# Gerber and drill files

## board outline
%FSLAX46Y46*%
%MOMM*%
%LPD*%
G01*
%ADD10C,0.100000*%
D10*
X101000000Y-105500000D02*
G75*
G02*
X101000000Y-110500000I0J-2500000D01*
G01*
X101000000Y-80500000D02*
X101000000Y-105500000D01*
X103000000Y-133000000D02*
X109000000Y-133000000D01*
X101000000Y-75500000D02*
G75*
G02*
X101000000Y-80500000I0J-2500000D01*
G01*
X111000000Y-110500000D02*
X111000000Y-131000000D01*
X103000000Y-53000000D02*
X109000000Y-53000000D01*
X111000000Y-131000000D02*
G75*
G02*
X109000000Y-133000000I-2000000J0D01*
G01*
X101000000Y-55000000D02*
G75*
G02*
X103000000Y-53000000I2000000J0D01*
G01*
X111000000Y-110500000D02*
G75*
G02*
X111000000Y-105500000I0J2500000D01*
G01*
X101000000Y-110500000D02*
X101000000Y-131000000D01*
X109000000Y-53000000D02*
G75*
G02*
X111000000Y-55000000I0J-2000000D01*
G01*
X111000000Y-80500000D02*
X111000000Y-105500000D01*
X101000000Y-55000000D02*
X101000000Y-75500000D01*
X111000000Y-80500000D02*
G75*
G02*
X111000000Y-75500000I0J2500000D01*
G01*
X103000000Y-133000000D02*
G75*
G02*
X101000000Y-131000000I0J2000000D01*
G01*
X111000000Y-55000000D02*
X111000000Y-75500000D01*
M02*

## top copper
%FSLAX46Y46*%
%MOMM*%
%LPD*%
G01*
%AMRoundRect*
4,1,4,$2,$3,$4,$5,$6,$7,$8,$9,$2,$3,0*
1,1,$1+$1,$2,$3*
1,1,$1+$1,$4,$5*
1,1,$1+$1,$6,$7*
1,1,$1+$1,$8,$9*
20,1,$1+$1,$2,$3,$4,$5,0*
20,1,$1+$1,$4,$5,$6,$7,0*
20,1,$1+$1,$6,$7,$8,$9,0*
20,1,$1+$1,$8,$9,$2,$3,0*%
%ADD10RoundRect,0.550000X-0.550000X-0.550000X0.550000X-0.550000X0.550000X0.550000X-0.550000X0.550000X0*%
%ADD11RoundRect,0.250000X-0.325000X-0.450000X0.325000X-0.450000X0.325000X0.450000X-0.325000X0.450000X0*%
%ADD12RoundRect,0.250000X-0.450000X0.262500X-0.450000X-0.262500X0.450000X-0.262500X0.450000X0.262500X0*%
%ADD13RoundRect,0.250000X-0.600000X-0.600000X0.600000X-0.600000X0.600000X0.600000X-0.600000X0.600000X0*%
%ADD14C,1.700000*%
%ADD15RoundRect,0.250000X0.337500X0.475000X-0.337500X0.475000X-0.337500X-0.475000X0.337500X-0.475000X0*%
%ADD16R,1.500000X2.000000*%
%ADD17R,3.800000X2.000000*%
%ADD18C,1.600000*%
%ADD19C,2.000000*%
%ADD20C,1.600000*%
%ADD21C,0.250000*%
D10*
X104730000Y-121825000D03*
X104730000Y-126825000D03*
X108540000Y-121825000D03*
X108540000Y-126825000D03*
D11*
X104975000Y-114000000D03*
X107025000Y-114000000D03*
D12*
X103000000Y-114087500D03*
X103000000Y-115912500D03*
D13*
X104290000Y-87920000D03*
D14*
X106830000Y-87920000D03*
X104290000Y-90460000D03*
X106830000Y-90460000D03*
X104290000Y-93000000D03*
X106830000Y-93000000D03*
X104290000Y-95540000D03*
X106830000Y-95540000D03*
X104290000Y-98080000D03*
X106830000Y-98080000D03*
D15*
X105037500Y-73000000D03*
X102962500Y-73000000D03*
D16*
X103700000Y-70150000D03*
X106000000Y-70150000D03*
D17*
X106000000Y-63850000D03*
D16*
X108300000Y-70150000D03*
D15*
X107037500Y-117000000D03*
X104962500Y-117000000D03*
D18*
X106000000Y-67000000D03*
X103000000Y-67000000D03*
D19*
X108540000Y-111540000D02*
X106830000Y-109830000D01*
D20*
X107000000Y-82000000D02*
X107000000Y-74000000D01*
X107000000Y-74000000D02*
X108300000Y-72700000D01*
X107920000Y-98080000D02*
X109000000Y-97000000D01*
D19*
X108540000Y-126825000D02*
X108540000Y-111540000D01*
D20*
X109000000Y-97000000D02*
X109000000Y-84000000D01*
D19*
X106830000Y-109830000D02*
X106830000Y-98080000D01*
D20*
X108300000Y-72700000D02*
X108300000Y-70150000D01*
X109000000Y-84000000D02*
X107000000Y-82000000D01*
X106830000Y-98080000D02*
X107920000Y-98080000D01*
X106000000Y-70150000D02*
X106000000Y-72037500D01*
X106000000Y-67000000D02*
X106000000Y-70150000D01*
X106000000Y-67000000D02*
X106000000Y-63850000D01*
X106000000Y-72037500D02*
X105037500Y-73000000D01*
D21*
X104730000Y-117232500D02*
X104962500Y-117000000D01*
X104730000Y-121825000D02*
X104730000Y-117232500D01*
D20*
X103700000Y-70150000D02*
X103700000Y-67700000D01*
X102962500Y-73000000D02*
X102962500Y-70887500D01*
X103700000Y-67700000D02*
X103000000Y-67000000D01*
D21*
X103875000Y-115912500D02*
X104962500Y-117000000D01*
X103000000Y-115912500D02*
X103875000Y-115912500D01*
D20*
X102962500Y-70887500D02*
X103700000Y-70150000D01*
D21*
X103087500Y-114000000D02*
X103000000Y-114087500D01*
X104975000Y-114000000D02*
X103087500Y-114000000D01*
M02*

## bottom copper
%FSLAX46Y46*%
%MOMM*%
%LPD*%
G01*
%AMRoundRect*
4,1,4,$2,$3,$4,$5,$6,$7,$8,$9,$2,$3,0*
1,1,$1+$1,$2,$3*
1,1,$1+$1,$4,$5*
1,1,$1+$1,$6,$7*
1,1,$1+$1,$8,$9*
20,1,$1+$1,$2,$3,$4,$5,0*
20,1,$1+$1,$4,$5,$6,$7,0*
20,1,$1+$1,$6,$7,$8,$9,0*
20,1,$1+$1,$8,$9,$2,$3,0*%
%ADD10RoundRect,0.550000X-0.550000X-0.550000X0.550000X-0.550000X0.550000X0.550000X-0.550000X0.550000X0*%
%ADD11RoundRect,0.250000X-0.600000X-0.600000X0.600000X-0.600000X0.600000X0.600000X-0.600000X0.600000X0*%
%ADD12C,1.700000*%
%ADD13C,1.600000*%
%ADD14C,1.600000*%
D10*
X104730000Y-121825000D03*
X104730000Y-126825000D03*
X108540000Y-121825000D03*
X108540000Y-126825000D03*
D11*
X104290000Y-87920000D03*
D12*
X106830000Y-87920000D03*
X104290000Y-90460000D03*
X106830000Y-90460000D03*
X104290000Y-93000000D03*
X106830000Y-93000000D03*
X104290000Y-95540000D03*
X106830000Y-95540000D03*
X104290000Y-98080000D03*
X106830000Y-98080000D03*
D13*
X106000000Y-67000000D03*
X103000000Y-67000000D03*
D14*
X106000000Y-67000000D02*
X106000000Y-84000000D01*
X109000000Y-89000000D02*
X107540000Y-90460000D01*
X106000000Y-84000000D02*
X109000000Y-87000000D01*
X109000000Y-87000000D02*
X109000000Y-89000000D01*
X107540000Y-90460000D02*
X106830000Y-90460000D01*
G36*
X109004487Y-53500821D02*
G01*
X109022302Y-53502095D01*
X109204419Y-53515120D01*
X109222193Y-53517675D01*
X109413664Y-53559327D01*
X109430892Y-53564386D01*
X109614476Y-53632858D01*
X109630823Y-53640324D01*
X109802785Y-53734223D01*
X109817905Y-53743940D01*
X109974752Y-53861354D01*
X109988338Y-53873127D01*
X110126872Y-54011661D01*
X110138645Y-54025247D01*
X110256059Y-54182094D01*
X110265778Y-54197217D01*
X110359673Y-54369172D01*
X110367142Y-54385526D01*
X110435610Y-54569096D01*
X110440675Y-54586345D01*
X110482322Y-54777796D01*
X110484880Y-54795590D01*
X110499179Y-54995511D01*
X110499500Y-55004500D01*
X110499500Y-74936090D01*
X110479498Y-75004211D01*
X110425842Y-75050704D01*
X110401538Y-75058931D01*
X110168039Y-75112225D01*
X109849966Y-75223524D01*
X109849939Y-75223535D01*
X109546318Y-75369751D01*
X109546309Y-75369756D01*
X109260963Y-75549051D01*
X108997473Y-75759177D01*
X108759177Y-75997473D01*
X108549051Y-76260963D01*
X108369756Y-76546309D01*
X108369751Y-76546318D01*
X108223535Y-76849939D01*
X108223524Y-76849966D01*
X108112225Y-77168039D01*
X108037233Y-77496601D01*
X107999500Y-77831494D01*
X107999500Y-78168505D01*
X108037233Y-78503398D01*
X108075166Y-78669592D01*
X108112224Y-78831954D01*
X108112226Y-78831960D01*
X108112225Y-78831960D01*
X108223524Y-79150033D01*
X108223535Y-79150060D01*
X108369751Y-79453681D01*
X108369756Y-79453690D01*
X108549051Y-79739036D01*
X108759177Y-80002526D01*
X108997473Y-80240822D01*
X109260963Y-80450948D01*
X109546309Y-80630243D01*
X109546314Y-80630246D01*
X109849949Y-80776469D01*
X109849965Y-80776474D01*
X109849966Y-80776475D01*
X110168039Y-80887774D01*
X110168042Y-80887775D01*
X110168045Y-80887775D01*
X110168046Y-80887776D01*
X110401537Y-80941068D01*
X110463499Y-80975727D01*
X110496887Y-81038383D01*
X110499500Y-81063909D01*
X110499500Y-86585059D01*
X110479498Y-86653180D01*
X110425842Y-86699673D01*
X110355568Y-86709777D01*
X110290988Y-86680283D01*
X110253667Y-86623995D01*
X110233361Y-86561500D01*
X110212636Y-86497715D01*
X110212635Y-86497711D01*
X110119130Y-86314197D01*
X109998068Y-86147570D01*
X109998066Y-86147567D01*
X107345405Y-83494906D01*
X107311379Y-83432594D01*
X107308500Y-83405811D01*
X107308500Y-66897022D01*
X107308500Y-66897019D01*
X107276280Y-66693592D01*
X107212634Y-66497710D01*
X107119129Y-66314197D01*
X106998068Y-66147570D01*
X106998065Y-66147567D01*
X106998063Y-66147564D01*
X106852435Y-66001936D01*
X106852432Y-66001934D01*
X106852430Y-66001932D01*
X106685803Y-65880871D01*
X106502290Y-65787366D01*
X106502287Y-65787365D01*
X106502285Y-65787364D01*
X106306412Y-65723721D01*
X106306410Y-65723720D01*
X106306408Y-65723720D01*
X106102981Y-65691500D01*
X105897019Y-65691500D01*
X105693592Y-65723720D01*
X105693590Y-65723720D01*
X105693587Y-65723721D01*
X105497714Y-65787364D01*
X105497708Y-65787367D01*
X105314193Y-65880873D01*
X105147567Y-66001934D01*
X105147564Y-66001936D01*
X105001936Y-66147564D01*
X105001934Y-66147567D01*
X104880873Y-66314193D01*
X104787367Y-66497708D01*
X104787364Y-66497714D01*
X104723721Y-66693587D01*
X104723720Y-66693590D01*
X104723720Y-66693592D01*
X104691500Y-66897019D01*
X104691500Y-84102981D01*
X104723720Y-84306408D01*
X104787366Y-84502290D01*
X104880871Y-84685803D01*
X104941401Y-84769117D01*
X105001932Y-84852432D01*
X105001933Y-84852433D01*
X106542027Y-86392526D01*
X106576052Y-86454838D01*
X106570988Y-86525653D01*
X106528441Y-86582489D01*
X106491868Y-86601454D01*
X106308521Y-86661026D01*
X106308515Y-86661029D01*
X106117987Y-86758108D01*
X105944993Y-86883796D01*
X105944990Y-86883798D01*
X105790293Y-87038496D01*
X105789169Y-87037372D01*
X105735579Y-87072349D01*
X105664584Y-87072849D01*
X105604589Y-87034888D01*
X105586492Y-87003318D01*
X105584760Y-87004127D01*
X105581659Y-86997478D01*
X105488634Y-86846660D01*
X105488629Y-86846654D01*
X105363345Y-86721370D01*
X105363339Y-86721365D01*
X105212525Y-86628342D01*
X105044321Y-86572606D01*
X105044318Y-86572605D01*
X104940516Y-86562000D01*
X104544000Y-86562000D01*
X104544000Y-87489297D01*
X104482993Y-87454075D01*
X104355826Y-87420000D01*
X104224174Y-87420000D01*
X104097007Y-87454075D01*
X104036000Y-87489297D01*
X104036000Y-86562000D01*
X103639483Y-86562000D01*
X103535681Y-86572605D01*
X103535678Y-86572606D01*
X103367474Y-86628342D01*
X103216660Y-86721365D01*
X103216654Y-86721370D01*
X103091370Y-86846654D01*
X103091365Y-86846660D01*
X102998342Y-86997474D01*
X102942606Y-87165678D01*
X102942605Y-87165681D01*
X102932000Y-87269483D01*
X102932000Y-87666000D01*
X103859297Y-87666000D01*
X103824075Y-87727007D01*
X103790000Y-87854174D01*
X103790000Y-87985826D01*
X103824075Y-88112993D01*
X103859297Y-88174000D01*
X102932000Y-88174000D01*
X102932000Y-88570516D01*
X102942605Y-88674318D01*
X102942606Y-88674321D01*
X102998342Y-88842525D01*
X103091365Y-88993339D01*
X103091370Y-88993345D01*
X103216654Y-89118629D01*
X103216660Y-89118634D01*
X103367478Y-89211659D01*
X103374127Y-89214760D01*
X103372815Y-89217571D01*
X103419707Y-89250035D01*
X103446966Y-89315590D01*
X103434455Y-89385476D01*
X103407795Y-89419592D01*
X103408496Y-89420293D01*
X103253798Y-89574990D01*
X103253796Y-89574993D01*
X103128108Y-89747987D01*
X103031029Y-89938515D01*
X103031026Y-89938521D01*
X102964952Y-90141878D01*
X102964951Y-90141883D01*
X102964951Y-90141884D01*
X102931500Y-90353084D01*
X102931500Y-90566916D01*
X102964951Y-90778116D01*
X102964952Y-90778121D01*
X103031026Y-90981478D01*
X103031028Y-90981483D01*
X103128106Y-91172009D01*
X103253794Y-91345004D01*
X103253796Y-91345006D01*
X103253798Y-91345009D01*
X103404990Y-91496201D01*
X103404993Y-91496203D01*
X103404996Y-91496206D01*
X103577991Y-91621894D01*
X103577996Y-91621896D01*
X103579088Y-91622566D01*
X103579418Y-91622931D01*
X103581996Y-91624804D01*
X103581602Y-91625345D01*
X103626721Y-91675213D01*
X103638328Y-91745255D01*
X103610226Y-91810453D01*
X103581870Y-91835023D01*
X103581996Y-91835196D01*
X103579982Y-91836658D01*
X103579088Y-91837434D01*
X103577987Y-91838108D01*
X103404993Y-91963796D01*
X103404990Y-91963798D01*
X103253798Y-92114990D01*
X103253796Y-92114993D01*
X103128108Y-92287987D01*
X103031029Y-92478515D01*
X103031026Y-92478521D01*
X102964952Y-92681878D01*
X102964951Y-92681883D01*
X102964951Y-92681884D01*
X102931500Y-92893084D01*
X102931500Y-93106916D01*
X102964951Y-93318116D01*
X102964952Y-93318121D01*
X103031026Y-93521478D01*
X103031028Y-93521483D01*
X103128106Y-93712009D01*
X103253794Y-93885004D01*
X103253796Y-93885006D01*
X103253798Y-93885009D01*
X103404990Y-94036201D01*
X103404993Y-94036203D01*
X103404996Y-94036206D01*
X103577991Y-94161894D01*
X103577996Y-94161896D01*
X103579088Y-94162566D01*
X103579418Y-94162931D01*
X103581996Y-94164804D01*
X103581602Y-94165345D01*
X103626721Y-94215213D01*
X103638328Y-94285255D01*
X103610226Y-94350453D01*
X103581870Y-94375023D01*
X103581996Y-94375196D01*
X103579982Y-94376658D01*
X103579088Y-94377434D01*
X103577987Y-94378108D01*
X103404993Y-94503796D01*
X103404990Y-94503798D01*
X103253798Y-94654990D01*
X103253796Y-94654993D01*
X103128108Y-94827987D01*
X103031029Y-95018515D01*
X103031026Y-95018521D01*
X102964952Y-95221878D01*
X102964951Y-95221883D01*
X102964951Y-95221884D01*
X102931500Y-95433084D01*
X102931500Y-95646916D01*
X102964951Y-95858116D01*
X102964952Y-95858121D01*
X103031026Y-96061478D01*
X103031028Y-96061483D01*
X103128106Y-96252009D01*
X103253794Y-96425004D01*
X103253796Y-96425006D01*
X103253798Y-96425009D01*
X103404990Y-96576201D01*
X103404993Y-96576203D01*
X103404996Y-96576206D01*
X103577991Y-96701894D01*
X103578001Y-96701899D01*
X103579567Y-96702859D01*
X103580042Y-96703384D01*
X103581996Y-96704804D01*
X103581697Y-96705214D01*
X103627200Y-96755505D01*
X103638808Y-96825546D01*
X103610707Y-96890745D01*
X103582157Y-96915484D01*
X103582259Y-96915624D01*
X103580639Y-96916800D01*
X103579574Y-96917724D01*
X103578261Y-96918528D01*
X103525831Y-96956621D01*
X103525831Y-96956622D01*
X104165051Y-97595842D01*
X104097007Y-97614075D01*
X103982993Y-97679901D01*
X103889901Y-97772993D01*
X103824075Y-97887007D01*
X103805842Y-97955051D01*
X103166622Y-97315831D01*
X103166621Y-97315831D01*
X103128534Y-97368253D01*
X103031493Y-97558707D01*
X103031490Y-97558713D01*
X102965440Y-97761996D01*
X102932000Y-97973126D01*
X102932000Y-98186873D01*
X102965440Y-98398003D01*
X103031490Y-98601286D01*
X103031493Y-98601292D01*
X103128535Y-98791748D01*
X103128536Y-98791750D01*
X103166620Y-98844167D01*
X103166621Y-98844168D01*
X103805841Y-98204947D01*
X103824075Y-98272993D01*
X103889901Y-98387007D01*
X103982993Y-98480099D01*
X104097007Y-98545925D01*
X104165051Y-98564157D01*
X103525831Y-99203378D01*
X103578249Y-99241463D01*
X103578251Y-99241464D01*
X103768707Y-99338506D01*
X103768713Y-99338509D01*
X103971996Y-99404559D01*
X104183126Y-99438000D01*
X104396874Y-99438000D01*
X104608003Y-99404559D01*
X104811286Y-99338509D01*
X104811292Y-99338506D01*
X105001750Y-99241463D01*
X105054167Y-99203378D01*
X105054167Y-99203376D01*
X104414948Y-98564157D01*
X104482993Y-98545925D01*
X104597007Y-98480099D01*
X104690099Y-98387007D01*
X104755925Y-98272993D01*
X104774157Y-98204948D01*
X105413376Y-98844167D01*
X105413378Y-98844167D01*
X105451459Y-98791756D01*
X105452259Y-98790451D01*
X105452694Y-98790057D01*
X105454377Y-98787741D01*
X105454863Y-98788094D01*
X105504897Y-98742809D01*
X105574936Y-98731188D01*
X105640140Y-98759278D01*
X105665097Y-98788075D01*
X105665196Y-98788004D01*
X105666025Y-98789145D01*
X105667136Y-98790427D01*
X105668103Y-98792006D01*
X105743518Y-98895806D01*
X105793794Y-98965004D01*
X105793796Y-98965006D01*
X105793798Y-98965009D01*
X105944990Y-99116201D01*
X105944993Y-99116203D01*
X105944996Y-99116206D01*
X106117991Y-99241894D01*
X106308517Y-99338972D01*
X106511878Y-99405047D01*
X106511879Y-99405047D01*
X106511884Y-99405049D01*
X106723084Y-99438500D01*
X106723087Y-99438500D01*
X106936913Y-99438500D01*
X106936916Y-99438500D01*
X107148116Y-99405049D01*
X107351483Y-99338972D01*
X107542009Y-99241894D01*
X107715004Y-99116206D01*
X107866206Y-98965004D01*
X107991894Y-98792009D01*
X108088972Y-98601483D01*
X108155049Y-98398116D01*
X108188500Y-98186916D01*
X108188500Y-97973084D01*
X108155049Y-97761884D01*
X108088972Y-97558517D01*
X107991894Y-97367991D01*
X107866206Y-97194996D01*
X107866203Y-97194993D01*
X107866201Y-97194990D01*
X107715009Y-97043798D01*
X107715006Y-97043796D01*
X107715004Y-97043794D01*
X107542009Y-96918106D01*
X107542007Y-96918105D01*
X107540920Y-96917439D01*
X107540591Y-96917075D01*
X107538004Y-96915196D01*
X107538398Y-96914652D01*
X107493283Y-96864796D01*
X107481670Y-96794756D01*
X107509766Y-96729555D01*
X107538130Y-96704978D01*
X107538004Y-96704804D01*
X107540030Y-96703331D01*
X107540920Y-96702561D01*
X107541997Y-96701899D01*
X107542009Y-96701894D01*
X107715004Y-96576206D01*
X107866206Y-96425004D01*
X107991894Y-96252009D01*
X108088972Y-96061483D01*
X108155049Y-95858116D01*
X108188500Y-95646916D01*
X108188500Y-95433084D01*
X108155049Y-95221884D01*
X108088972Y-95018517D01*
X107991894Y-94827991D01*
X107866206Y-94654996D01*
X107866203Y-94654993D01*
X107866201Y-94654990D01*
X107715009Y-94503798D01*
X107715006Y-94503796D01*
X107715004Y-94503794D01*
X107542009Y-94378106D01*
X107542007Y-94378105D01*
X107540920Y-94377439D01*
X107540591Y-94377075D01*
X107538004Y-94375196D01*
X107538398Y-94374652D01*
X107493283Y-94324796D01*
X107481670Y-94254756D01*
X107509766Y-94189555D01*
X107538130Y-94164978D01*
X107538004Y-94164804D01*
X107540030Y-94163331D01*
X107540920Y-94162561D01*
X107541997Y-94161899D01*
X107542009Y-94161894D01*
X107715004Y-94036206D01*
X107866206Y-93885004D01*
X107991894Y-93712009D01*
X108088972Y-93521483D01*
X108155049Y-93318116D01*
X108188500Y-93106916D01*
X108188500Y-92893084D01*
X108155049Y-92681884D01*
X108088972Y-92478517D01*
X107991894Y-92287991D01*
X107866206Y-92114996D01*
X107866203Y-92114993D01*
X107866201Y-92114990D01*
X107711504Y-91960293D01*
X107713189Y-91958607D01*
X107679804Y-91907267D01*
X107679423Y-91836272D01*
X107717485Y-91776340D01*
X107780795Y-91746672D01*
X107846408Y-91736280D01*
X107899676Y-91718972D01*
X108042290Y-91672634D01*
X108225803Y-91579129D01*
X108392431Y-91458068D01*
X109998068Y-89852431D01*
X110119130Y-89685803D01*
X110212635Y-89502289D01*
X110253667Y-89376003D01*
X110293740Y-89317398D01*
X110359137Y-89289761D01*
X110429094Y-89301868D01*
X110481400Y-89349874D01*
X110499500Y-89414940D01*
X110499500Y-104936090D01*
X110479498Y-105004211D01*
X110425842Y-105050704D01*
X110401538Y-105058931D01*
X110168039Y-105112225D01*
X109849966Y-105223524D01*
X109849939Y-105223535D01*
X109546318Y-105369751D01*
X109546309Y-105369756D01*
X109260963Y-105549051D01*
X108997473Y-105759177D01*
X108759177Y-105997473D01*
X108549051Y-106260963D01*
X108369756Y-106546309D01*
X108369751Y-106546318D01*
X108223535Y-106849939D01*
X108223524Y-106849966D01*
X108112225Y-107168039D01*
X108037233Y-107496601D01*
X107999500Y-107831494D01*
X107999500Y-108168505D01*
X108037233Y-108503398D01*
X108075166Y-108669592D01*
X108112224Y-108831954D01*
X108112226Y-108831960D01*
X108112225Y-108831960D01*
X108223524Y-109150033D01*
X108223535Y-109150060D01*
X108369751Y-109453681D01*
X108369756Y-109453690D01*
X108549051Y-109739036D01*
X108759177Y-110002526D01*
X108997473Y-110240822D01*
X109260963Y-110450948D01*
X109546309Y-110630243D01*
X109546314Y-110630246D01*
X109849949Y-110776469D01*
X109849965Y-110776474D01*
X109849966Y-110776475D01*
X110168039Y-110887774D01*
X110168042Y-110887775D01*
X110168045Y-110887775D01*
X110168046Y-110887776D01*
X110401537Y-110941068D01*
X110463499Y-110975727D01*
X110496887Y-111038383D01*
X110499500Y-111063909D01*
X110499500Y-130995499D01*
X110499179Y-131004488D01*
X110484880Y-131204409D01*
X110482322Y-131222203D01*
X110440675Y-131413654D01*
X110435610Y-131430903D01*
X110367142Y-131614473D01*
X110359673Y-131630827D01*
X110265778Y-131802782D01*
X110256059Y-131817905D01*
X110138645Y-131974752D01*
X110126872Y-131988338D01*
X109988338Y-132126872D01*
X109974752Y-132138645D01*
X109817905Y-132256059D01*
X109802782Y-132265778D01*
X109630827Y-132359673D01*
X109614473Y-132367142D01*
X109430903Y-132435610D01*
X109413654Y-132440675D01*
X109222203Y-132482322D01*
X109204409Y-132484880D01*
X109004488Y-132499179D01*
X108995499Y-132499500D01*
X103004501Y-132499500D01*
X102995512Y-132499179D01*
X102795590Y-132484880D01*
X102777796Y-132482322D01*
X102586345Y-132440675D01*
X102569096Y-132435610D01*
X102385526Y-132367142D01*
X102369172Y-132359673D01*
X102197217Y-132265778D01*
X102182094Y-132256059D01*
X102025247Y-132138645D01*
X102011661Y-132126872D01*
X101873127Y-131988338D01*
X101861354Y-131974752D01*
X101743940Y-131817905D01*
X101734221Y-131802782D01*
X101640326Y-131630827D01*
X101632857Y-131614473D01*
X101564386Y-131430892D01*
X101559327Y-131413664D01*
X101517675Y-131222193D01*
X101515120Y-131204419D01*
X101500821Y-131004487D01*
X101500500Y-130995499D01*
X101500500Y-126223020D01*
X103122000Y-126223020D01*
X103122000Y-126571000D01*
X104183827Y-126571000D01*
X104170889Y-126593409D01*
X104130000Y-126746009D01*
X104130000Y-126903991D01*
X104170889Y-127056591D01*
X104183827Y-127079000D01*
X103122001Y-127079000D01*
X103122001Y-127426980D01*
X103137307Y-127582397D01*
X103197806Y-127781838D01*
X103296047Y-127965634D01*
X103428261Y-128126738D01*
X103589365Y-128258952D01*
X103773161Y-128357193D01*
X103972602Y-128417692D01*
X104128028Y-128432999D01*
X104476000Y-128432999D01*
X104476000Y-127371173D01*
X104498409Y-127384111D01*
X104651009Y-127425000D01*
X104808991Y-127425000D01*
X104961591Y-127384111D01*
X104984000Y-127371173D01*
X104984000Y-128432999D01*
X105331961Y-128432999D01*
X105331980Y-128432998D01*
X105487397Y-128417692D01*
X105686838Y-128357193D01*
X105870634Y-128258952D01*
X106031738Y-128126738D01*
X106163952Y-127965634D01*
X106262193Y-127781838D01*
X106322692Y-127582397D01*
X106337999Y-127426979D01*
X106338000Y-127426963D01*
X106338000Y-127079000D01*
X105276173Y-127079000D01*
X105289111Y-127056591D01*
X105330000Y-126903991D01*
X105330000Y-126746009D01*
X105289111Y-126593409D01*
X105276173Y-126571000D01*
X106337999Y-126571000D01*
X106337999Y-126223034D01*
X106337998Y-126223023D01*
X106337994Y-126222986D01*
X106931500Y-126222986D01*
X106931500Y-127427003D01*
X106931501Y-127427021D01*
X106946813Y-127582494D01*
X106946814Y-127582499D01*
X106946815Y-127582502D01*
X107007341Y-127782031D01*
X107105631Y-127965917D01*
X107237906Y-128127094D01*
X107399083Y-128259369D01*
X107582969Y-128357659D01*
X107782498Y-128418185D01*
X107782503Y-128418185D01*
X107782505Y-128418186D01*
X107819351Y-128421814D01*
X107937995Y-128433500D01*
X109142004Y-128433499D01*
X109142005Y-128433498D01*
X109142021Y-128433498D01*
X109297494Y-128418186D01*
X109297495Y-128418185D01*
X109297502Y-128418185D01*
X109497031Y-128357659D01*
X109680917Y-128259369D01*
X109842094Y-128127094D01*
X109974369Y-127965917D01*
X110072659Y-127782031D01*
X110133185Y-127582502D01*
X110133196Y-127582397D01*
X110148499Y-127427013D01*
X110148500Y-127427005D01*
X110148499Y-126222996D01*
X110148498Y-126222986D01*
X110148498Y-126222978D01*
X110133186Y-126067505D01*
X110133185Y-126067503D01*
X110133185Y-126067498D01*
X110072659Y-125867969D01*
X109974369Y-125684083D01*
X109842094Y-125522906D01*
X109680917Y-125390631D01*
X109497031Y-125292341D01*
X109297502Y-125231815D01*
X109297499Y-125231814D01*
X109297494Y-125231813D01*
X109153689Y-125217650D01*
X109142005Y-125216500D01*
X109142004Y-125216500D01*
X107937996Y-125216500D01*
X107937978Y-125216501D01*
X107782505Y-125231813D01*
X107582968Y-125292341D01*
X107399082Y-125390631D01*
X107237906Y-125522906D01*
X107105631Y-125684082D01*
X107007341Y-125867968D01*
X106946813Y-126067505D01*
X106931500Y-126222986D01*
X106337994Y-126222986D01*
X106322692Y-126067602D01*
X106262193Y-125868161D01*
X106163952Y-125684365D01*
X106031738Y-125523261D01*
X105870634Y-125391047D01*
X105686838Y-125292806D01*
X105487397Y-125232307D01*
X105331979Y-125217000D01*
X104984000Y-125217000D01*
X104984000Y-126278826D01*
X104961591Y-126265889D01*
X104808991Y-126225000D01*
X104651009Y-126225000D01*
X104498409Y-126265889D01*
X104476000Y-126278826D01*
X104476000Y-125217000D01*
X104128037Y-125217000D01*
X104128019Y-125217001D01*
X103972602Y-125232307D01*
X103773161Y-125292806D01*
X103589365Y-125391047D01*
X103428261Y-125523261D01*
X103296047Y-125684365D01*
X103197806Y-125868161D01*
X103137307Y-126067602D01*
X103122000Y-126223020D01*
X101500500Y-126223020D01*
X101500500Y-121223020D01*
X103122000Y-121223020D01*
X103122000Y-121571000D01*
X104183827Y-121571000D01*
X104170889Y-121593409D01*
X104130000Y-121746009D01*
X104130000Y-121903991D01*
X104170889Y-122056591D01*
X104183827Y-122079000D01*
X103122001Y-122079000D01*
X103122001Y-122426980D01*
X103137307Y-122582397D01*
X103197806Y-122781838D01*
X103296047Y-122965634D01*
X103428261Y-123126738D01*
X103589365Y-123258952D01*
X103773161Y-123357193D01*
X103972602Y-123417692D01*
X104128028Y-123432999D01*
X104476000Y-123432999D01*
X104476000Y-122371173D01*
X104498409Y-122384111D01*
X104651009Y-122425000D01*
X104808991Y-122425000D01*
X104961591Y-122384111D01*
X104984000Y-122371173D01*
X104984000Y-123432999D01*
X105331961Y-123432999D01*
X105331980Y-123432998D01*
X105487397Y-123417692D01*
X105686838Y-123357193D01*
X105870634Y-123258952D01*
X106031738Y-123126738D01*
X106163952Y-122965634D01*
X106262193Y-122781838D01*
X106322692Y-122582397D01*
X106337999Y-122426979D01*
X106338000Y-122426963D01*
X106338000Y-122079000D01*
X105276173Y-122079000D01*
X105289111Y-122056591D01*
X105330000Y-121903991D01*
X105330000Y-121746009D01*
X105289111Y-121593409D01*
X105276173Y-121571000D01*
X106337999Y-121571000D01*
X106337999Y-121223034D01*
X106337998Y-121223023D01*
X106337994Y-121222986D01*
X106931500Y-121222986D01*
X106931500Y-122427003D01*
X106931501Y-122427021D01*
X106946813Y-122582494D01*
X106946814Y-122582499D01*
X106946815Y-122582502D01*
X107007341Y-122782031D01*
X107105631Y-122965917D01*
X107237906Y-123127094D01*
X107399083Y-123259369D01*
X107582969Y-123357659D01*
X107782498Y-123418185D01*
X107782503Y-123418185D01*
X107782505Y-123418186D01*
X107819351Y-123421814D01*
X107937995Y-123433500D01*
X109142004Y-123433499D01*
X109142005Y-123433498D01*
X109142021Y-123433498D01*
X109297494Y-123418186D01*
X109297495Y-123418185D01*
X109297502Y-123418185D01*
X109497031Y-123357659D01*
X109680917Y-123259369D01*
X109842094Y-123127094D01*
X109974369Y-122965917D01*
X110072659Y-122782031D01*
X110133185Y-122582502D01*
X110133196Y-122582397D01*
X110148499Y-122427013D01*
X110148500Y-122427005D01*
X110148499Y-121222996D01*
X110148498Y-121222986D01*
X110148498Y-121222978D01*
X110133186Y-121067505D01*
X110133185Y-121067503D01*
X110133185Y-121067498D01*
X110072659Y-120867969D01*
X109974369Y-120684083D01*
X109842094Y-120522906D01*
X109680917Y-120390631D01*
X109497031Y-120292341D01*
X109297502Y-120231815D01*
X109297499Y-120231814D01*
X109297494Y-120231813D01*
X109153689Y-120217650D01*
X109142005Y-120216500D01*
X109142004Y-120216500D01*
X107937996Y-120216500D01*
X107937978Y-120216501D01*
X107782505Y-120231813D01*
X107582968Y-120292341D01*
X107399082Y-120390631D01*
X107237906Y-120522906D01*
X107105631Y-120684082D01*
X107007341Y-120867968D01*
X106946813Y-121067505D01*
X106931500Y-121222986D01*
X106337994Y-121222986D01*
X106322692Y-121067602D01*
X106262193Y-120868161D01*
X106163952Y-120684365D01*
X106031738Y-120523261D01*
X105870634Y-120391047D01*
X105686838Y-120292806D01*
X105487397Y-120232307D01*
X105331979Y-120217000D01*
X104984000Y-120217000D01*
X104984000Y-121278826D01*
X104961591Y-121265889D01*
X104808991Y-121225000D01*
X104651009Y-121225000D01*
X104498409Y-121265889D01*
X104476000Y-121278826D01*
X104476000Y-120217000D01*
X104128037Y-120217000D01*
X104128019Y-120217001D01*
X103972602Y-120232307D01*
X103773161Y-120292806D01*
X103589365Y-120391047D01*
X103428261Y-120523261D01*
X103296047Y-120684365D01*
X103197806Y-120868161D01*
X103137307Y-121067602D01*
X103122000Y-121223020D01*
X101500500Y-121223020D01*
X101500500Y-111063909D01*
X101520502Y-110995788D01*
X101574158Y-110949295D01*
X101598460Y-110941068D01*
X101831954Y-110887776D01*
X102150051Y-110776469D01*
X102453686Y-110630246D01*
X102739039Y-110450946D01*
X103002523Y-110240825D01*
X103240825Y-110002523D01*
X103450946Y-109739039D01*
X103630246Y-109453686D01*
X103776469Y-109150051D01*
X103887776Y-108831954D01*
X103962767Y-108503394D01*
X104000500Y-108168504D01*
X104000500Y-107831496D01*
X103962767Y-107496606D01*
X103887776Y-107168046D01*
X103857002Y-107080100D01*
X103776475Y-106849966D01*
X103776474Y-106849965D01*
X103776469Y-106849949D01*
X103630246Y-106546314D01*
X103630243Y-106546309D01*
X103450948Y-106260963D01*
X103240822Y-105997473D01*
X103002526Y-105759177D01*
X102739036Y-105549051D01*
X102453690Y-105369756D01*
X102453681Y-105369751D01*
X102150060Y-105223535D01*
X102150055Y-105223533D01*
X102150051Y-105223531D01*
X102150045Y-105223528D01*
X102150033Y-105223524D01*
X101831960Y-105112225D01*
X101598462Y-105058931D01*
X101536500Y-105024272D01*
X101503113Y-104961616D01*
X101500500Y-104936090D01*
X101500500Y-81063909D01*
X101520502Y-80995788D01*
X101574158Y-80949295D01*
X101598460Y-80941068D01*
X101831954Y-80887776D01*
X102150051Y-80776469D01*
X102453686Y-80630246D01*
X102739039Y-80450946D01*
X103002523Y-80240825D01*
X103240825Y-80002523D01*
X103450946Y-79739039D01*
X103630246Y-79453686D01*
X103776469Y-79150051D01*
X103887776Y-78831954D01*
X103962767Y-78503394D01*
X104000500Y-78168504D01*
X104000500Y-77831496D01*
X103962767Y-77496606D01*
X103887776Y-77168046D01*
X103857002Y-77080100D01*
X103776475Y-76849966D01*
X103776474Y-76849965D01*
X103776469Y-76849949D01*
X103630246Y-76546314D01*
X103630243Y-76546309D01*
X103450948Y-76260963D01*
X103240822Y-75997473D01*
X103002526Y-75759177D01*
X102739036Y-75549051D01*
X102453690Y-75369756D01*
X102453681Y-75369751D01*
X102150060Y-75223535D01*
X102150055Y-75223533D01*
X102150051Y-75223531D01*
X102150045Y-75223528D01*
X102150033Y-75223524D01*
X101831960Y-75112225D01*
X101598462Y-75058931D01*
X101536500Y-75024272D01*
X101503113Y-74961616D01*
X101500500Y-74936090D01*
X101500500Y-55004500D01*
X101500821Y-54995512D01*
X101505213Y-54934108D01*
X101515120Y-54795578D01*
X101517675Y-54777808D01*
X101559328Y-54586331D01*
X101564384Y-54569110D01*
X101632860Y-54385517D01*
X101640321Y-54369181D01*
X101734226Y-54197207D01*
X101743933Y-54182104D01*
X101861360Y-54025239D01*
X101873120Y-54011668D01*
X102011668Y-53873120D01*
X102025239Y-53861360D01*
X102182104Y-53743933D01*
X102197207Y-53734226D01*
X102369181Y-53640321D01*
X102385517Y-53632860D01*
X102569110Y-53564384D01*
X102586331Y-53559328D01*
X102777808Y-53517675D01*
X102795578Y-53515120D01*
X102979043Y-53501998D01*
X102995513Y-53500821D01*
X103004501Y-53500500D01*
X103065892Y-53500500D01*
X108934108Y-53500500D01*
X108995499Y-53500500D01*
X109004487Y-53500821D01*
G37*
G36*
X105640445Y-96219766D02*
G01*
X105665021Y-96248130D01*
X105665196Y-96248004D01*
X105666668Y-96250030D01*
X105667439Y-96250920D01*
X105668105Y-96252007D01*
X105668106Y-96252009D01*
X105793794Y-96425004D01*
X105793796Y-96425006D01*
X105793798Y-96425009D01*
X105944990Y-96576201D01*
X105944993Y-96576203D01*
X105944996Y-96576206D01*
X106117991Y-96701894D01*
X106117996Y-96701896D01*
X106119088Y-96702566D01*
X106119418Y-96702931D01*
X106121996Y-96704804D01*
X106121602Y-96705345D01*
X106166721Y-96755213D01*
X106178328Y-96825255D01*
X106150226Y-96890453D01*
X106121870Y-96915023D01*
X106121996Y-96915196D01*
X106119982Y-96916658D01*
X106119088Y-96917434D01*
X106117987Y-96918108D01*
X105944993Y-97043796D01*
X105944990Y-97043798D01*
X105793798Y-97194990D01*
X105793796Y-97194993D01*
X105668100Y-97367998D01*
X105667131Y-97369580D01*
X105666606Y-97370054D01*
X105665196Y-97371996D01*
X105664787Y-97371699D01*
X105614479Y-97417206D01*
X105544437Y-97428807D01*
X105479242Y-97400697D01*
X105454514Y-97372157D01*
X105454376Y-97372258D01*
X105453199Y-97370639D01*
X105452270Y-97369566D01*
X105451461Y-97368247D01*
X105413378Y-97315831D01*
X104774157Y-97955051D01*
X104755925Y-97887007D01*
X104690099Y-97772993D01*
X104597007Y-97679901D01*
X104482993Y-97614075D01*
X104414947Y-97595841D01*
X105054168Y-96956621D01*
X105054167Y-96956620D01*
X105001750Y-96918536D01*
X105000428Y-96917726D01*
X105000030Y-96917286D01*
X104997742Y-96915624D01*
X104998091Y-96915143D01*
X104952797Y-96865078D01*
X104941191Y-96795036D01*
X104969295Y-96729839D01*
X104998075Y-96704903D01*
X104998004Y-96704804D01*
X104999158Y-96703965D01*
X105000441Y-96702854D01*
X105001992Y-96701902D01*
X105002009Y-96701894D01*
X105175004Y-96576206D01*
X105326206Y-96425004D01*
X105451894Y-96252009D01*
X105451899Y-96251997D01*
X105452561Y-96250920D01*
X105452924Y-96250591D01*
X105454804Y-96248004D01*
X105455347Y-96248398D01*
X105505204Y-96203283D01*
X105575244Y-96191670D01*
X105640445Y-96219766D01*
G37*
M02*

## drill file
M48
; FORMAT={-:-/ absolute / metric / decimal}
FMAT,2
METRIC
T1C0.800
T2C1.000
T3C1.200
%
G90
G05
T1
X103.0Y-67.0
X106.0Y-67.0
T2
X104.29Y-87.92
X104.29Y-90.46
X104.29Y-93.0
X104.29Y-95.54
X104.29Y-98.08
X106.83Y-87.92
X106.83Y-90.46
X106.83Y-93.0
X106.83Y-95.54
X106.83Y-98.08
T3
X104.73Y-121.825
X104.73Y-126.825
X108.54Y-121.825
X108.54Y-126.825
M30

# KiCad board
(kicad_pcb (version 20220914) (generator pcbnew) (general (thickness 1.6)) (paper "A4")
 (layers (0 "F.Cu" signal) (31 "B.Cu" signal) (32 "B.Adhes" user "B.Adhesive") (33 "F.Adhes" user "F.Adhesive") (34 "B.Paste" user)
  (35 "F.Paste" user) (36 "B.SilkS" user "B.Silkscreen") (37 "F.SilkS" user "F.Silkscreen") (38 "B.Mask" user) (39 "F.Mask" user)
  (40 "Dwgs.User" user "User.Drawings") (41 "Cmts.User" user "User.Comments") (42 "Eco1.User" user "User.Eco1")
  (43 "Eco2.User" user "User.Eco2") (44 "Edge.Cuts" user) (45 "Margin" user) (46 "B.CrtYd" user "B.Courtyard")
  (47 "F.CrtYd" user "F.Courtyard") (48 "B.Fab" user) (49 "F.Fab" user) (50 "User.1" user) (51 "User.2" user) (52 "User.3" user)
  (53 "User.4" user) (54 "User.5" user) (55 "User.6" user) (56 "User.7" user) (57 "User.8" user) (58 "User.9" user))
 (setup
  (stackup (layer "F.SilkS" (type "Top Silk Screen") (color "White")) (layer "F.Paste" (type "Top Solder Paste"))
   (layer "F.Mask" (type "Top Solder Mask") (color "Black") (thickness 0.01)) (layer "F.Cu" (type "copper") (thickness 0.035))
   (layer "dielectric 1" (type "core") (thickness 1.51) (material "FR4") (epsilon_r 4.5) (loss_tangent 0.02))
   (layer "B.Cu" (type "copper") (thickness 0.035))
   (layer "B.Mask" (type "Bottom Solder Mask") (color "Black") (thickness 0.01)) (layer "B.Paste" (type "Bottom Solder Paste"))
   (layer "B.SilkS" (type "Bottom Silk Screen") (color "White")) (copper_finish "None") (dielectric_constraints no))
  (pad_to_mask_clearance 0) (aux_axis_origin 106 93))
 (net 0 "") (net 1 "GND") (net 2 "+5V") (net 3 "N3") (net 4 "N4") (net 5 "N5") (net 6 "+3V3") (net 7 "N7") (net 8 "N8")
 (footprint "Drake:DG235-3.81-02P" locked (layer "F.Cu") (at 104.73 121.825)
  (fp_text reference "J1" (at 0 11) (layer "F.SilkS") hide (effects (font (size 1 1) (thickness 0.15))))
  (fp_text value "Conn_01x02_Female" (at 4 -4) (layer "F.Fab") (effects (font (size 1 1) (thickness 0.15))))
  (pad "1" thru_hole roundrect locked (at 0 0) (size 2.2 2.2) (drill 1.2) (layers *.Cu *.Mask) (roundrect_rratio 0.25) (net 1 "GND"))
  (pad "1" thru_hole roundrect locked (at 0 5) (size 2.2 2.2) (drill 1.2) (layers *.Cu *.Mask) (roundrect_rratio 0.25) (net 1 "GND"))
  (pad "2" thru_hole roundrect locked (at 3.81 0) (size 2.2 2.2) (drill 1.2) (layers *.Cu *.Mask) (roundrect_rratio 0.25) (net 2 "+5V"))
  (pad "2" thru_hole roundrect locked (at 3.81 5) (size 2.2 2.2) (drill 1.2) (layers *.Cu *.Mask) (roundrect_rratio 0.25) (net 2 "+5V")))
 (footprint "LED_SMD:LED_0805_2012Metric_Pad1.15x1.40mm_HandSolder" (layer "F.Cu") (at 106 114)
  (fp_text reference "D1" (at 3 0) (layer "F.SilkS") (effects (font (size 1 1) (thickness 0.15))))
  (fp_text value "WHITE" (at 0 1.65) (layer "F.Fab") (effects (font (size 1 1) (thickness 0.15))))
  (pad "1" smd roundrect (at -1.025 0) (size 1.15 1.4) (layers "F.Cu" "F.Paste" "F.Mask") (roundrect_rratio 0.217391) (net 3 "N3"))
  (pad "2" smd roundrect (at 1.025 0) (size 1.15 1.4) (layers "F.Cu" "F.Paste" "F.Mask") (roundrect_rratio 0.217391) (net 2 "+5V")))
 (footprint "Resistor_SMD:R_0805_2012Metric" (layer "F.Cu") (at 103 115 -90)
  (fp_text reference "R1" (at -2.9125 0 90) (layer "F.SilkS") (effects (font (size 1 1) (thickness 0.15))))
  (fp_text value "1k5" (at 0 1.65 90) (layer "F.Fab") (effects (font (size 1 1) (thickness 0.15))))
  (pad "1" smd roundrect (at -0.9125 0 270) (size 1.025 1.4) (layers "F.Cu" "F.Paste" "F.Mask") (roundrect_rratio 0.243902) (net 3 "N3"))
  (pad "2" smd roundrect (at 0.9125 0 270) (size 1.025 1.4) (layers "F.Cu" "F.Paste" "F.Mask") (roundrect_rratio 0.243902) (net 1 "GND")))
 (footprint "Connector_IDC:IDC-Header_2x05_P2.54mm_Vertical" (layer "F.Cu") (at 104.29 87.92)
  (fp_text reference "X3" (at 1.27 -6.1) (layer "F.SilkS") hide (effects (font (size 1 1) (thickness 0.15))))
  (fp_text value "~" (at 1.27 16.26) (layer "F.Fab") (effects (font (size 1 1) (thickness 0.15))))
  (pad "1" thru_hole roundrect (at 0 0) (size 1.7 1.7) (drill 1) (layers *.Cu *.Mask) (roundrect_rratio 0.147059) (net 1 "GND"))
  (pad "2" thru_hole circle (at 2.54 0) (size 1.7 1.7) (drill 1) (layers *.Cu *.Mask) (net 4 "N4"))
  (pad "3" thru_hole circle (at 0 2.54) (size 1.7 1.7) (drill 1) (layers *.Cu *.Mask) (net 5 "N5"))
  (pad "4" thru_hole circle (at 2.54 2.54) (size 1.7 1.7) (drill 1) (layers *.Cu *.Mask) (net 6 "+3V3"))
  (pad "5" thru_hole circle (at 0 5.08) (size 1.7 1.7) (drill 1) (layers *.Cu *.Mask))
  (pad "6" thru_hole circle (at 2.54 5.08) (size 1.7 1.7) (drill 1) (layers *.Cu *.Mask))
  (pad "7" thru_hole circle (at 0 7.62) (size 1.7 1.7) (drill 1) (layers *.Cu *.Mask) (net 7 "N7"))
  (pad "8" thru_hole circle (at 2.54 7.62) (size 1.7 1.7) (drill 1) (layers *.Cu *.Mask) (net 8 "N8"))
  (pad "9" thru_hole circle (at 0 10.16) (size 1.7 1.7) (drill 1) (layers *.Cu *.Mask) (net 1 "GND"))
  (pad "10" thru_hole circle (at 2.54 10.16) (size 1.7 1.7) (drill 1) (layers *.Cu *.Mask) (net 2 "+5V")))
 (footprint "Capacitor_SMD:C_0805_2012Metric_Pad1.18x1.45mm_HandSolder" (layer "F.Cu") (at 104 73 180)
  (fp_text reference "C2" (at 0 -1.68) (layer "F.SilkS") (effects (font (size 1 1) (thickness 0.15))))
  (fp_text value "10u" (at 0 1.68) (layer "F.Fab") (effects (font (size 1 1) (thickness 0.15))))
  (pad "1" smd roundrect (at -1.0375 0 180) (size 1.175 1.45) (layers "F.Cu" "F.Paste" "F.Mask") (roundrect_rratio 0.212766) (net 6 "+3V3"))
  (pad "2" smd roundrect (at 1.0375 0 180) (size 1.175 1.45) (layers "F.Cu" "F.Paste" "F.Mask") (roundrect_rratio 0.212766) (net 1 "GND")))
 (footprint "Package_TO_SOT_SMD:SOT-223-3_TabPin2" (layer "F.Cu") (at 106 67 90)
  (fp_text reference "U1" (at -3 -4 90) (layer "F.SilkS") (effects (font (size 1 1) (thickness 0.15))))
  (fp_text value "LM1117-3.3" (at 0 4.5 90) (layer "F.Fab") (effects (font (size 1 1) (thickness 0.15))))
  (pad "1" smd rect (at -3.15 -2.3 90) (size 2 1.5) (layers "F.Cu" "F.Paste" "F.Mask") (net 1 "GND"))
  (pad "2" smd rect (at -3.15 0 90) (size 2 1.5) (layers "F.Cu" "F.Paste" "F.Mask") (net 6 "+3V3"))
  (pad "2" smd rect (at 3.15 0 90) (size 2 3.8) (layers "F.Cu" "F.Paste" "F.Mask") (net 6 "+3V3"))
  (pad "3" smd rect (at -3.15 2.3 90) (size 2 1.5) (layers "F.Cu" "F.Paste" "F.Mask") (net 2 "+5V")))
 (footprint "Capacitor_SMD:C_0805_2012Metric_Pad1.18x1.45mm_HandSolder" (layer "F.Cu") (at 106 117 180)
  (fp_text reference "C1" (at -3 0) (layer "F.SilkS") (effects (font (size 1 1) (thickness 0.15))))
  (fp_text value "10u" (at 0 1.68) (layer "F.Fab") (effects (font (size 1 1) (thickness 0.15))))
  (pad "1" smd roundrect (at -1.0375 0 180) (size 1.175 1.45) (layers "F.Cu" "F.Paste" "F.Mask") (roundrect_rratio 0.212766) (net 2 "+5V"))
  (pad "2" smd roundrect (at 1.0375 0 180) (size 1.175 1.45) (layers "F.Cu" "F.Paste" "F.Mask") (roundrect_rratio 0.212766) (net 1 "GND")))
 (gr_arc (start 101 105.5) (mid 103.5 108) (end 101 110.5) (stroke (width 0.1) (type default)) (layer "Edge.Cuts"))
 (gr_line (start 101 80.5) (end 101 105.5) (stroke (width 0.1) (type default)) (layer "Edge.Cuts"))
 (gr_line (start 103 133) (end 109 133) (stroke (width 0.1) (type default)) (layer "Edge.Cuts"))
 (gr_arc (start 101 75.5) (mid 103.5 78) (end 101 80.5) (stroke (width 0.1) (type default)) (layer "Edge.Cuts"))
 (gr_line (start 111 110.5) (end 111 131) (stroke (width 0.1) (type default)) (layer "Edge.Cuts"))
 (gr_line (start 103 53) (end 109 53) (stroke (width 0.1) (type default)) (layer "Edge.Cuts"))
 (gr_arc (start 111 131) (mid 110.414214 132.414214) (end 109 133) (stroke (width 0.1) (type default)) (layer "Edge.Cuts"))
 (gr_arc (start 101 55) (mid 101.585786 53.585786) (end 103 53) (stroke (width 0.1) (type default)) (layer "Edge.Cuts"))
 (gr_arc (start 111 110.5) (mid 108.5 108) (end 111 105.5) (stroke (width 0.1) (type default)) (layer "Edge.Cuts"))
 (gr_line (start 101 110.5) (end 101 131) (stroke (width 0.1) (type default)) (layer "Edge.Cuts"))
 (gr_arc (start 109 53) (mid 110.414214 53.585786) (end 111 55) (stroke (width 0.1) (type default)) (layer "Edge.Cuts"))
 (gr_line (start 111 80.5) (end 111 105.5) (stroke (width 0.1) (type default)) (layer "Edge.Cuts"))
 (gr_line (start 101 55) (end 101 75.5) (stroke (width 0.1) (type default)) (layer "Edge.Cuts"))
 (gr_arc (start 111 80.5) (mid 108.5 78) (end 111 75.5) (stroke (width 0.1) (type default)) (layer "Edge.Cuts"))
 (gr_arc (start 103 133) (mid 101.585786 132.414214) (end 101 131) (stroke (width 0.1) (type default)) (layer "Edge.Cuts"))
 (gr_line (start 111 55) (end 111 75.5) (stroke (width 0.1) (type default)) (layer "Edge.Cuts"))
 (segment (start 108.54 111.54) (end 106.83 109.83) (width 2) (layer "F.Cu") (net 2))
 (segment (start 107 82) (end 107 74) (width 1.6) (layer "F.Cu") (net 2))
 (segment (start 107 74) (end 108.3 72.7) (width 1.6) (layer "F.Cu") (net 2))
 (segment (start 107.92 98.08) (end 109 97) (width 1.6) (layer "F.Cu") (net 2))
 (segment (start 108.54 126.825) (end 108.54 111.54) (width 2) (layer "F.Cu") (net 2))
 (segment (start 109 97) (end 109 84) (width 1.6) (layer "F.Cu") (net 2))
 (segment (start 106.83 109.83) (end 106.83 98.08) (width 2) (layer "F.Cu") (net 2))
 (segment (start 108.3 72.7) (end 108.3 70.15) (width 1.6) (layer "F.Cu") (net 2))
 (segment (start 109 84) (end 107 82) (width 1.6) (layer "F.Cu") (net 2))
 (segment (start 106.83 98.08) (end 107.92 98.08) (width 1.6) (layer "F.Cu") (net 2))
 (segment (start 106 70.15) (end 106 72.0375) (width 1.6) (layer "F.Cu") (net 6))
 (segment (start 106 67) (end 106 70.15) (width 1.6) (layer "F.Cu") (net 6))
 (segment (start 106 67) (end 106 63.85) (width 1.6) (layer "F.Cu") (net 6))
 (segment (start 106 72.0375) (end 105.0375 73) (width 1.6) (layer "F.Cu") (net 6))
 (via (at 106 67) (size 1.6) (drill 0.8) (layers "F.Cu" "B.Cu") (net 6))
 (segment (start 106 67) (end 106 84) (width 1.6) (layer "B.Cu") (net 6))
 (segment (start 109 89) (end 107.54 90.46) (width 1.6) (layer "B.Cu") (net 6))
 (segment (start 106 84) (end 109 87) (width 1.6) (layer "B.Cu") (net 6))
 (segment (start 109 87) (end 109 89) (width 1.6) (layer "B.Cu") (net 6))
 (segment (start 107.54 90.46) (end 106.83 90.46) (width 1.6) (layer "B.Cu") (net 6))
 (segment (start 104.73 117.2325) (end 104.9625 117) (width 0.25) (layer "F.Cu") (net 1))
 (segment (start 104.73 121.825) (end 104.73 117.2325) (width 0.25) (layer "F.Cu") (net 1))
 (segment (start 103.7 70.15) (end 103.7 67.7) (width 1.6) (layer "F.Cu") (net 1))
 (segment (start 102.9625 73) (end 102.9625 70.8875) (width 1.6) (layer "F.Cu") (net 1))
 (segment (start 103.7 67.7) (end 103 67) (width 1.6) (layer "F.Cu") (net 1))
 (segment (start 103.875 115.9125) (end 104.9625 117) (width 0.25) (layer "F.Cu") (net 1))
 (segment (start 103 115.9125) (end 103.875 115.9125) (width 0.25) (layer "F.Cu") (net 1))
 (segment (start 102.9625 70.8875) (end 103.7 70.15) (width 1.6) (layer "F.Cu") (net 1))
 (via (at 103 67) (size 1.6) (drill 0.8) (layers "F.Cu" "B.Cu") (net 1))
 (segment (start 103.0875 114) (end 103 114.0875) (width 0.25) (layer "F.Cu") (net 3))
 (segment (start 104.975 114) (end 103.0875 114) (width 0.25) (layer "F.Cu") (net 3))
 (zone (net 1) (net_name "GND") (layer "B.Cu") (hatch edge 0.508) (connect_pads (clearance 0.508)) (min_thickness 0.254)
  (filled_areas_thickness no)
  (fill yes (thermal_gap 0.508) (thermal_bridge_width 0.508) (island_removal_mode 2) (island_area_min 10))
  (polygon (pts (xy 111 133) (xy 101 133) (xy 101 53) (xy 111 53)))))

